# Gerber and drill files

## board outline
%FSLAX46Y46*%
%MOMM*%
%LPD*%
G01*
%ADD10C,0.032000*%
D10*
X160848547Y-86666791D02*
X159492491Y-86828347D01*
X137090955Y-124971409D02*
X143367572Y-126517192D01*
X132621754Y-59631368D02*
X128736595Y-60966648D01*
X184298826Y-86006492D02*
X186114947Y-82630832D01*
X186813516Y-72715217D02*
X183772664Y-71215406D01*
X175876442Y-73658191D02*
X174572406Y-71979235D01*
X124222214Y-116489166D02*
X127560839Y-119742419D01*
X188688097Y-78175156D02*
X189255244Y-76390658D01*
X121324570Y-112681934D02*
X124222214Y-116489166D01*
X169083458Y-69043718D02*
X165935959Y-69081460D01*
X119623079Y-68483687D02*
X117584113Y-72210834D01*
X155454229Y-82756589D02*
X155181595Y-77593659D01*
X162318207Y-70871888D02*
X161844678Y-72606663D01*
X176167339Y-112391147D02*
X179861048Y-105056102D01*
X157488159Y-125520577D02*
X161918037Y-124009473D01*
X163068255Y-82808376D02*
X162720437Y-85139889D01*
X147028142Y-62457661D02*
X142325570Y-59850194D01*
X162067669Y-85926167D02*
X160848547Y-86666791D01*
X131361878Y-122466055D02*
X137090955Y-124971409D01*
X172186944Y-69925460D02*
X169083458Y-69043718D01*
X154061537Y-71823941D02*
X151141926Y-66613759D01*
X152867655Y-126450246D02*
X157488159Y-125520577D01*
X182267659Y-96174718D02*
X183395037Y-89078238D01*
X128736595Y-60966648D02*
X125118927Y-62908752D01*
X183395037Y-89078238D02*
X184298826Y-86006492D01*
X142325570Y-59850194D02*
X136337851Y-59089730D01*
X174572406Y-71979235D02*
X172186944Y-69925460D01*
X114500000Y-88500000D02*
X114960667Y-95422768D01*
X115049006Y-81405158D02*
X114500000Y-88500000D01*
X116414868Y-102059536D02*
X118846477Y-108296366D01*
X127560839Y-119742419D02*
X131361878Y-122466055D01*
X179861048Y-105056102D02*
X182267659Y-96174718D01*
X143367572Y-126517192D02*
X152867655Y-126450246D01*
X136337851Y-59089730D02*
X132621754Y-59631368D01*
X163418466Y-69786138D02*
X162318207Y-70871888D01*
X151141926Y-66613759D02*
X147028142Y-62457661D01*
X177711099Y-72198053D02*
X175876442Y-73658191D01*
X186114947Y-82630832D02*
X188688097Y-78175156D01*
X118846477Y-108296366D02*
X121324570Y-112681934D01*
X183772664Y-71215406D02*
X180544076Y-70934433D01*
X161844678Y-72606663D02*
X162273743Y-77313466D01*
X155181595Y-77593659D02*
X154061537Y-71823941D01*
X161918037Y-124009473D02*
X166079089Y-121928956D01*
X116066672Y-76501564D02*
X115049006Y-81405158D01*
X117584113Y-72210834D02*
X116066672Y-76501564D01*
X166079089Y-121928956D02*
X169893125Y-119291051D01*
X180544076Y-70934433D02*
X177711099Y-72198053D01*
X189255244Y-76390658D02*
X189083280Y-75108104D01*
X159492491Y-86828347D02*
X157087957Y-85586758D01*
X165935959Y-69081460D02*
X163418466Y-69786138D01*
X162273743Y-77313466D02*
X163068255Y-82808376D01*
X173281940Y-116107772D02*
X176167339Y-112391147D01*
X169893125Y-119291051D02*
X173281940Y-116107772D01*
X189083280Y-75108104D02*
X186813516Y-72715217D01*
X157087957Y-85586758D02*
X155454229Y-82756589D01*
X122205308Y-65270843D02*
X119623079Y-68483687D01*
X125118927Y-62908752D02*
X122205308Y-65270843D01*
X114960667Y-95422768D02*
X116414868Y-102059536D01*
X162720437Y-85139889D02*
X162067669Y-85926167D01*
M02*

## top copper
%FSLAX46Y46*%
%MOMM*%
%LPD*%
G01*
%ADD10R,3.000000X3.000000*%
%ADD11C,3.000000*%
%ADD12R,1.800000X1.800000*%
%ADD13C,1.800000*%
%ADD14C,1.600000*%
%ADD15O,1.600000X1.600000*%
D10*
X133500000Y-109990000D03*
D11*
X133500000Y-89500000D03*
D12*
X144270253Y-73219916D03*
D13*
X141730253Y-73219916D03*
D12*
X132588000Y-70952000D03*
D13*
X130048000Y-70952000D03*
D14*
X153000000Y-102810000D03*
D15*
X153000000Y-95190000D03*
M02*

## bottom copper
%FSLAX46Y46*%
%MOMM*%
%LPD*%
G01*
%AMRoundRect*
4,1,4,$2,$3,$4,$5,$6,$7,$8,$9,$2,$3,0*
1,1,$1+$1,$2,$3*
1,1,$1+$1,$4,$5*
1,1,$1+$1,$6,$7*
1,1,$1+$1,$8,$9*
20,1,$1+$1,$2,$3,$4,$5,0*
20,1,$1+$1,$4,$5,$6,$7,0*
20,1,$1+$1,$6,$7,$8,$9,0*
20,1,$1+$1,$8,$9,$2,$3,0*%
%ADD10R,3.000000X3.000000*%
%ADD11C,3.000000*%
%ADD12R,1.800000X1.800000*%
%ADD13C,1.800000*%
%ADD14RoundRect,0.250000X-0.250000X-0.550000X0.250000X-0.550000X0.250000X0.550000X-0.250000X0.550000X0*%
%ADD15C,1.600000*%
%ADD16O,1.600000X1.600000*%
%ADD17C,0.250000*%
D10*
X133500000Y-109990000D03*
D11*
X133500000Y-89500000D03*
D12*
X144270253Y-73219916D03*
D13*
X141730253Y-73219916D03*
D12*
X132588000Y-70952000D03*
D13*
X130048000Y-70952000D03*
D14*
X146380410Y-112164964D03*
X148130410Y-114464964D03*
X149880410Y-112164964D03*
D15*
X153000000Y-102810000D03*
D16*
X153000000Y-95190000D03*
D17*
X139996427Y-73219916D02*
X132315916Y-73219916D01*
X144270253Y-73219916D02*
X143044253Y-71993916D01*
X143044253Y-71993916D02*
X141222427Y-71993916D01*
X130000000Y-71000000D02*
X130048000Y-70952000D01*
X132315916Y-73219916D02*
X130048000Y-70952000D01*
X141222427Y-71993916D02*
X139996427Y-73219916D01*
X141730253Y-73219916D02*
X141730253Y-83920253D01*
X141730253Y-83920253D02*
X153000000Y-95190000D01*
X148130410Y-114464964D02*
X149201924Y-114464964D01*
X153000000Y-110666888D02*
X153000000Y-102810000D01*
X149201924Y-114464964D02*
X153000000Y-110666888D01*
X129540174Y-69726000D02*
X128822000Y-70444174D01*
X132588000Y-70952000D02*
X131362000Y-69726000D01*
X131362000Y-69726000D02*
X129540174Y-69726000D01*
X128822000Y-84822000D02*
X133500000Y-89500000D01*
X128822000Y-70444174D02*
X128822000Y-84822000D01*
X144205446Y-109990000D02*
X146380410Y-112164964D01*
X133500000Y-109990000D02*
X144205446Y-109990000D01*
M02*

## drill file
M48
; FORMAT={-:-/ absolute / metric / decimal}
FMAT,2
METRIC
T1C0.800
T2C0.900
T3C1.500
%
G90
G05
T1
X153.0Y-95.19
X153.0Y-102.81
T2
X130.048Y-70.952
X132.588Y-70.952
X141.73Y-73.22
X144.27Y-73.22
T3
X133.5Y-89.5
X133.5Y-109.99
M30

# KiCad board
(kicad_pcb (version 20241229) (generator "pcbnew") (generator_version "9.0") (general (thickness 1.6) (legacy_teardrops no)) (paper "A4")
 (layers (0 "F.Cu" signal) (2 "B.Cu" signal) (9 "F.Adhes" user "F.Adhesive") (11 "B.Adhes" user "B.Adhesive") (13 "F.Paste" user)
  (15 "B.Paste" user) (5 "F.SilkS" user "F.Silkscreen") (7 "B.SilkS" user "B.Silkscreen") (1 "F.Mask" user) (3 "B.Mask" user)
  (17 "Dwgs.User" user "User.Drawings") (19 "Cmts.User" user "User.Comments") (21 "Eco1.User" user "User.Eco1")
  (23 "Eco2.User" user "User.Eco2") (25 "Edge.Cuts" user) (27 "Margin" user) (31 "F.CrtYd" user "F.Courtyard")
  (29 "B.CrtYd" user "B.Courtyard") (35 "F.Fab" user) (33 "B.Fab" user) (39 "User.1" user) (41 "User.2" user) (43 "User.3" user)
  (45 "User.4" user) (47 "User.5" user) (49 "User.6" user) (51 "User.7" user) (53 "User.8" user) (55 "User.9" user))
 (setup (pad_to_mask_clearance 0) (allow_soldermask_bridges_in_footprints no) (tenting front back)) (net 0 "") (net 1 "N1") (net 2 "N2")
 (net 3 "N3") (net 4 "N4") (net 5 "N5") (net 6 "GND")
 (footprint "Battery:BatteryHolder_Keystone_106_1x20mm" (layer "B.Cu") (at 133.5 109.99 90)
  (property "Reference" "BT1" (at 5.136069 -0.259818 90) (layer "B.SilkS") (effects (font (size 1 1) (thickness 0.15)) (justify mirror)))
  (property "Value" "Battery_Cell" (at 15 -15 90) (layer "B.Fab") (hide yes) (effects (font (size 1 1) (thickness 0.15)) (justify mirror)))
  (pad "1" thru_hole rect (at 0 0 90) (size 3 3) (drill 1.5) (layers "*.Cu" "*.Mask") (remove_unused_layers no) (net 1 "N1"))
  (pad "2" thru_hole circle (at 20.49 0 90) (size 3 3) (drill 1.5) (layers "*.Cu" "*.Mask") (remove_unused_layers no) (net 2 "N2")))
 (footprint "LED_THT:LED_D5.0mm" (layer "B.Cu") (at 144.270253 73.219916 180)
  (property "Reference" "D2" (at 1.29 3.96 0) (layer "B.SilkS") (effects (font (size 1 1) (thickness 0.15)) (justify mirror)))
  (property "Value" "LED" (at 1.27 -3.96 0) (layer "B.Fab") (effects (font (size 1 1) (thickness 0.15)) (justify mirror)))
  (pad "1" thru_hole rect (at 0 0 180) (size 1.8 1.8) (drill 0.9) (layers "*.Cu" "*.Mask") (remove_unused_layers no) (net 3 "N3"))
  (pad "2" thru_hole circle (at 2.54 0 180) (size 1.8 1.8) (drill 0.9) (layers "*.Cu" "*.Mask") (remove_unused_layers no) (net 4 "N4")))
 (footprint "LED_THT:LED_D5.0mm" (layer "B.Cu") (at 132.588 70.952 180)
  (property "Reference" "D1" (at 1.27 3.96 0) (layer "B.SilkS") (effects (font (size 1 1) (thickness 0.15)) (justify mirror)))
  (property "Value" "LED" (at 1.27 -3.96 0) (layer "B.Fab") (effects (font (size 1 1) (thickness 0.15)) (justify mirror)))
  (pad "1" thru_hole rect (at 0 0 180) (size 1.8 1.8) (drill 0.9) (layers "*.Cu" "*.Mask") (remove_unused_layers no) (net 2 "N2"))
  (pad "2" thru_hole circle (at 2.54 0 180) (size 1.8 1.8) (drill 0.9) (layers "*.Cu" "*.Mask") (remove_unused_layers no) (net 3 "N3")))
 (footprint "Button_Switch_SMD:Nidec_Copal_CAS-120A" (layer "B.Cu") (at 148.13041 113.314964 -90)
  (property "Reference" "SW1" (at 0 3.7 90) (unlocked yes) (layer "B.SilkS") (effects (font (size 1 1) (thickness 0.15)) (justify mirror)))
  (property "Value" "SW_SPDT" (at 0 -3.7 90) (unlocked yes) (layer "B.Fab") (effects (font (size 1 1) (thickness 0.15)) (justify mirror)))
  (pad "1" smd roundrect (at -1.15 1.75) (size 1 1.6) (layers "B.Cu" "B.Mask" "B.Paste") (roundrect_rratio 0.25) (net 1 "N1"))
  (pad "2" smd roundrect (at 1.15 0) (size 1 1.6) (layers "B.Cu" "B.Mask" "B.Paste") (roundrect_rratio 0.25) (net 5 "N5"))
  (pad "3" smd roundrect (at -1.15 -1.75) (size 1 1.6) (layers "B.Cu" "B.Mask" "B.Paste") (roundrect_rratio 0.25) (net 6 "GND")))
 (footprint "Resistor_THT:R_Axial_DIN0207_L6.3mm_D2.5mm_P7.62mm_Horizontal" (layer "B.Cu") (at 153 102.81 90)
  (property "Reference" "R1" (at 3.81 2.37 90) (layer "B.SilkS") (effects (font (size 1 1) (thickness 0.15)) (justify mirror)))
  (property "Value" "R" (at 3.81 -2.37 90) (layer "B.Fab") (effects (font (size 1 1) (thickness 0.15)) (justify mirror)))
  (pad "1" thru_hole circle (at 0 0 90) (size 1.6 1.6) (drill 0.8) (layers "*.Cu" "*.Mask") (remove_unused_layers no) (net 5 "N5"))
  (pad "2" thru_hole oval (at 7.62 0 90) (size 1.6 1.6) (drill 0.8) (layers "*.Cu" "*.Mask") (remove_unused_layers no) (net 4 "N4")))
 (gr_line (start 160.848547 86.666791) (end 159.492491 86.828347) (stroke (width 0.032) (type default)) (layer "Edge.Cuts"))
 (gr_line (start 137.090955 124.971409) (end 143.367572 126.517192) (stroke (width 0.032) (type default)) (layer "Edge.Cuts"))
 (gr_line (start 132.621754 59.631368) (end 128.736595 60.966648) (stroke (width 0.032) (type default)) (layer "Edge.Cuts"))
 (gr_line (start 184.298826 86.006492) (end 186.114947 82.630832) (stroke (width 0.032) (type default)) (layer "Edge.Cuts"))
 (gr_line (start 186.813516 72.715217) (end 183.772664 71.215406) (stroke (width 0.032) (type default)) (layer "Edge.Cuts"))
 (gr_line (start 175.876442 73.658191) (end 174.572406 71.979235) (stroke (width 0.032) (type default)) (layer "Edge.Cuts"))
 (gr_line (start 124.222214 116.489166) (end 127.560839 119.742419) (stroke (width 0.032) (type default)) (layer "Edge.Cuts"))
 (gr_line (start 188.688097 78.175156) (end 189.255244 76.390658) (stroke (width 0.032) (type default)) (layer "Edge.Cuts"))
 (gr_line (start 121.32457 112.681934) (end 124.222214 116.489166) (stroke (width 0.032) (type default)) (layer "Edge.Cuts"))
 (gr_line (start 169.083458 69.043718) (end 165.935959 69.08146) (stroke (width 0.032) (type default)) (layer "Edge.Cuts"))
 (gr_line (start 119.623079 68.483687) (end 117.584113 72.210834) (stroke (width 0.032) (type default)) (layer "Edge.Cuts"))
 (gr_line (start 155.454229 82.756589) (end 155.181595 77.593659) (stroke (width 0.032) (type default)) (layer "Edge.Cuts"))
 (gr_line (start 162.318207 70.871888) (end 161.844678 72.606663) (stroke (width 0.032) (type default)) (layer "Edge.Cuts"))
 (gr_line (start 176.167339 112.391147) (end 179.861048 105.056102) (stroke (width 0.032) (type default)) (layer "Edge.Cuts"))
 (gr_line (start 157.488159 125.520577) (end 161.918037 124.009473) (stroke (width 0.032) (type default)) (layer "Edge.Cuts"))
 (gr_line (start 163.068255 82.808376) (end 162.720437 85.139889) (stroke (width 0.032) (type default)) (layer "Edge.Cuts"))
 (gr_line (start 147.028142 62.457661) (end 142.32557 59.850194) (stroke (width 0.032) (type default)) (layer "Edge.Cuts"))
 (gr_line (start 162.067669 85.926167) (end 160.848547 86.666791) (stroke (width 0.032) (type default)) (layer "Edge.Cuts"))
 (gr_line (start 131.361878 122.466055) (end 137.090955 124.971409) (stroke (width 0.032) (type default)) (layer "Edge.Cuts"))
 (gr_line (start 172.186944 69.92546) (end 169.083458 69.043718) (stroke (width 0.032) (type default)) (layer "Edge.Cuts"))
 (gr_line (start 154.061537 71.823941) (end 151.141926 66.613759) (stroke (width 0.032) (type default)) (layer "Edge.Cuts"))
 (gr_line (start 152.867655 126.450246) (end 157.488159 125.520577) (stroke (width 0.032) (type default)) (layer "Edge.Cuts"))
 (gr_line (start 182.267659 96.174718) (end 183.395037 89.078238) (stroke (width 0.032) (type default)) (layer "Edge.Cuts"))
 (gr_line (start 128.736595 60.966648) (end 125.118927 62.908752) (stroke (width 0.032) (type default)) (layer "Edge.Cuts"))
 (gr_line (start 183.395037 89.078238) (end 184.298826 86.006492) (stroke (width 0.032) (type default)) (layer "Edge.Cuts"))
 (gr_line (start 142.32557 59.850194) (end 136.337851 59.08973) (stroke (width 0.032) (type default)) (layer "Edge.Cuts"))
 (gr_line (start 174.572406 71.979235) (end 172.186944 69.92546) (stroke (width 0.032) (type default)) (layer "Edge.Cuts"))
 (gr_line (start 114.5 88.5) (end 114.960667 95.422768) (stroke (width 0.032) (type default)) (layer "Edge.Cuts"))
 (gr_line (start 115.049006 81.405158) (end 114.5 88.5) (stroke (width 0.032) (type default)) (layer "Edge.Cuts"))
 (gr_line (start 116.414868 102.059536) (end 118.846477 108.296366) (stroke (width 0.032) (type default)) (layer "Edge.Cuts"))
 (gr_line (start 127.560839 119.742419) (end 131.361878 122.466055) (stroke (width 0.032) (type default)) (layer "Edge.Cuts"))
 (gr_line (start 179.861048 105.056102) (end 182.267659 96.174718) (stroke (width 0.032) (type default)) (layer "Edge.Cuts"))
 (gr_line (start 143.367572 126.517192) (end 152.867655 126.450246) (stroke (width 0.032) (type default)) (layer "Edge.Cuts"))
 (gr_line (start 136.337851 59.08973) (end 132.621754 59.631368) (stroke (width 0.032) (type default)) (layer "Edge.Cuts"))
 (gr_line (start 163.418466 69.786138) (end 162.318207 70.871888) (stroke (width 0.032) (type default)) (layer "Edge.Cuts"))
 (gr_line (start 151.141926 66.613759) (end 147.028142 62.457661) (stroke (width 0.032) (type default)) (layer "Edge.Cuts"))
 (gr_line (start 177.711099 72.198053) (end 175.876442 73.658191) (stroke (width 0.032) (type default)) (layer "Edge.Cuts"))
 (gr_line (start 186.114947 82.630832) (end 188.688097 78.175156) (stroke (width 0.032) (type default)) (layer "Edge.Cuts"))
 (gr_line (start 118.846477 108.296366) (end 121.32457 112.681934) (stroke (width 0.032) (type default)) (layer "Edge.Cuts"))
 (gr_line (start 183.772664 71.215406) (end 180.544076 70.934433) (stroke (width 0.032) (type default)) (layer "Edge.Cuts"))
 (gr_line (start 161.844678 72.606663) (end 162.273743 77.313466) (stroke (width 0.032) (type default)) (layer "Edge.Cuts"))
 (gr_line (start 155.181595 77.593659) (end 154.061537 71.823941) (stroke (width 0.032) (type default)) (layer "Edge.Cuts"))
 (gr_line (start 161.918037 124.009473) (end 166.079089 121.928956) (stroke (width 0.032) (type default)) (layer "Edge.Cuts"))
 (gr_line (start 116.066672 76.501564) (end 115.049006 81.405158) (stroke (width 0.032) (type default)) (layer "Edge.Cuts"))
 (gr_line (start 117.584113 72.210834) (end 116.066672 76.501564) (stroke (width 0.032) (type default)) (layer "Edge.Cuts"))
 (gr_line (start 166.079089 121.928956) (end 169.893125 119.291051) (stroke (width 0.032) (type default)) (layer "Edge.Cuts"))
 (gr_line (start 180.544076 70.934433) (end 177.711099 72.198053) (stroke (width 0.032) (type default)) (layer "Edge.Cuts"))
 (gr_line (start 189.255244 76.390658) (end 189.08328 75.108104) (stroke (width 0.032) (type default)) (layer "Edge.Cuts"))
 (gr_line (start 159.492491 86.828347) (end 157.087957 85.586758) (stroke (width 0.032) (type default)) (layer "Edge.Cuts"))
 (gr_line (start 165.935959 69.08146) (end 163.418466 69.786138) (stroke (width 0.032) (type default)) (layer "Edge.Cuts"))
 (gr_line (start 162.273743 77.313466) (end 163.068255 82.808376) (stroke (width 0.032) (type default)) (layer "Edge.Cuts"))
 (gr_line (start 173.28194 116.107772) (end 176.167339 112.391147) (stroke (width 0.032) (type default)) (layer "Edge.Cuts"))
 (gr_line (start 169.893125 119.291051) (end 173.28194 116.107772) (stroke (width 0.032) (type default)) (layer "Edge.Cuts"))
 (gr_line (start 189.08328 75.108104) (end 186.813516 72.715217) (stroke (width 0.032) (type default)) (layer "Edge.Cuts"))
 (gr_line (start 157.087957 85.586758) (end 155.454229 82.756589) (stroke (width 0.032) (type default)) (layer "Edge.Cuts"))
 (gr_line (start 122.205308 65.270843) (end 119.623079 68.483687) (stroke (width 0.032) (type default)) (layer "Edge.Cuts"))
 (gr_line (start 125.118927 62.908752) (end 122.205308 65.270843) (stroke (width 0.032) (type default)) (layer "Edge.Cuts"))
 (gr_line (start 114.960667 95.422768) (end 116.414868 102.059536) (stroke (width 0.032) (type default)) (layer "Edge.Cuts"))
 (gr_line (start 162.720437 85.139889) (end 162.067669 85.926167) (stroke (width 0.032) (type default)) (layer "Edge.Cuts"))
 (segment (start 139.996427 73.219916) (end 132.315916 73.219916) (width 0.25) (layer "B.Cu") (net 3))
 (segment (start 144.270253 73.219916) (end 143.044253 71.993916) (width 0.25) (layer "B.Cu") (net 3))
 (segment (start 143.044253 71.993916) (end 141.222427 71.993916) (width 0.25) (layer "B.Cu") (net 3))
 (segment (start 130 71) (end 130.048 70.952) (width 0.25) (layer "B.Cu") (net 3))
 (segment (start 132.315916 73.219916) (end 130.048 70.952) (width 0.25) (layer "B.Cu") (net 3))
 (segment (start 141.222427 71.993916) (end 139.996427 73.219916) (width 0.25) (layer "B.Cu") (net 3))
 (segment (start 141.730253 73.219916) (end 141.730253 83.920253) (width 0.25) (layer "B.Cu") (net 4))
 (segment (start 141.730253 83.920253) (end 153 95.19) (width 0.25) (layer "B.Cu") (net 4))
 (segment (start 148.13041 114.464964) (end 149.201924 114.464964) (width 0.25) (layer "B.Cu") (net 5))
 (segment (start 153 110.666888) (end 153 102.81) (width 0.25) (layer "B.Cu") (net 5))
 (segment (start 149.201924 114.464964) (end 153 110.666888) (width 0.25) (layer "B.Cu") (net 5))
 (segment (start 129.540174 69.726) (end 128.822 70.444174) (width 0.25) (layer "B.Cu") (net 2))
 (segment (start 132.588 70.952) (end 131.362 69.726) (width 0.25) (layer "B.Cu") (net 2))
 (segment (start 131.362 69.726) (end 129.540174 69.726) (width 0.25) (layer "B.Cu") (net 2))
 (segment (start 128.822 84.822) (end 133.5 89.5) (width 0.25) (layer "B.Cu") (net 2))
 (segment (start 128.822 70.444174) (end 128.822 84.822) (width 0.25) (layer "B.Cu") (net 2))
 (segment (start 144.205446 109.99) (end 146.38041 112.164964) (width 0.25) (layer "B.Cu") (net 1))
 (segment (start 133.5 109.99) (end 144.205446 109.99) (width 0.25) (layer "B.Cu") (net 1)))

